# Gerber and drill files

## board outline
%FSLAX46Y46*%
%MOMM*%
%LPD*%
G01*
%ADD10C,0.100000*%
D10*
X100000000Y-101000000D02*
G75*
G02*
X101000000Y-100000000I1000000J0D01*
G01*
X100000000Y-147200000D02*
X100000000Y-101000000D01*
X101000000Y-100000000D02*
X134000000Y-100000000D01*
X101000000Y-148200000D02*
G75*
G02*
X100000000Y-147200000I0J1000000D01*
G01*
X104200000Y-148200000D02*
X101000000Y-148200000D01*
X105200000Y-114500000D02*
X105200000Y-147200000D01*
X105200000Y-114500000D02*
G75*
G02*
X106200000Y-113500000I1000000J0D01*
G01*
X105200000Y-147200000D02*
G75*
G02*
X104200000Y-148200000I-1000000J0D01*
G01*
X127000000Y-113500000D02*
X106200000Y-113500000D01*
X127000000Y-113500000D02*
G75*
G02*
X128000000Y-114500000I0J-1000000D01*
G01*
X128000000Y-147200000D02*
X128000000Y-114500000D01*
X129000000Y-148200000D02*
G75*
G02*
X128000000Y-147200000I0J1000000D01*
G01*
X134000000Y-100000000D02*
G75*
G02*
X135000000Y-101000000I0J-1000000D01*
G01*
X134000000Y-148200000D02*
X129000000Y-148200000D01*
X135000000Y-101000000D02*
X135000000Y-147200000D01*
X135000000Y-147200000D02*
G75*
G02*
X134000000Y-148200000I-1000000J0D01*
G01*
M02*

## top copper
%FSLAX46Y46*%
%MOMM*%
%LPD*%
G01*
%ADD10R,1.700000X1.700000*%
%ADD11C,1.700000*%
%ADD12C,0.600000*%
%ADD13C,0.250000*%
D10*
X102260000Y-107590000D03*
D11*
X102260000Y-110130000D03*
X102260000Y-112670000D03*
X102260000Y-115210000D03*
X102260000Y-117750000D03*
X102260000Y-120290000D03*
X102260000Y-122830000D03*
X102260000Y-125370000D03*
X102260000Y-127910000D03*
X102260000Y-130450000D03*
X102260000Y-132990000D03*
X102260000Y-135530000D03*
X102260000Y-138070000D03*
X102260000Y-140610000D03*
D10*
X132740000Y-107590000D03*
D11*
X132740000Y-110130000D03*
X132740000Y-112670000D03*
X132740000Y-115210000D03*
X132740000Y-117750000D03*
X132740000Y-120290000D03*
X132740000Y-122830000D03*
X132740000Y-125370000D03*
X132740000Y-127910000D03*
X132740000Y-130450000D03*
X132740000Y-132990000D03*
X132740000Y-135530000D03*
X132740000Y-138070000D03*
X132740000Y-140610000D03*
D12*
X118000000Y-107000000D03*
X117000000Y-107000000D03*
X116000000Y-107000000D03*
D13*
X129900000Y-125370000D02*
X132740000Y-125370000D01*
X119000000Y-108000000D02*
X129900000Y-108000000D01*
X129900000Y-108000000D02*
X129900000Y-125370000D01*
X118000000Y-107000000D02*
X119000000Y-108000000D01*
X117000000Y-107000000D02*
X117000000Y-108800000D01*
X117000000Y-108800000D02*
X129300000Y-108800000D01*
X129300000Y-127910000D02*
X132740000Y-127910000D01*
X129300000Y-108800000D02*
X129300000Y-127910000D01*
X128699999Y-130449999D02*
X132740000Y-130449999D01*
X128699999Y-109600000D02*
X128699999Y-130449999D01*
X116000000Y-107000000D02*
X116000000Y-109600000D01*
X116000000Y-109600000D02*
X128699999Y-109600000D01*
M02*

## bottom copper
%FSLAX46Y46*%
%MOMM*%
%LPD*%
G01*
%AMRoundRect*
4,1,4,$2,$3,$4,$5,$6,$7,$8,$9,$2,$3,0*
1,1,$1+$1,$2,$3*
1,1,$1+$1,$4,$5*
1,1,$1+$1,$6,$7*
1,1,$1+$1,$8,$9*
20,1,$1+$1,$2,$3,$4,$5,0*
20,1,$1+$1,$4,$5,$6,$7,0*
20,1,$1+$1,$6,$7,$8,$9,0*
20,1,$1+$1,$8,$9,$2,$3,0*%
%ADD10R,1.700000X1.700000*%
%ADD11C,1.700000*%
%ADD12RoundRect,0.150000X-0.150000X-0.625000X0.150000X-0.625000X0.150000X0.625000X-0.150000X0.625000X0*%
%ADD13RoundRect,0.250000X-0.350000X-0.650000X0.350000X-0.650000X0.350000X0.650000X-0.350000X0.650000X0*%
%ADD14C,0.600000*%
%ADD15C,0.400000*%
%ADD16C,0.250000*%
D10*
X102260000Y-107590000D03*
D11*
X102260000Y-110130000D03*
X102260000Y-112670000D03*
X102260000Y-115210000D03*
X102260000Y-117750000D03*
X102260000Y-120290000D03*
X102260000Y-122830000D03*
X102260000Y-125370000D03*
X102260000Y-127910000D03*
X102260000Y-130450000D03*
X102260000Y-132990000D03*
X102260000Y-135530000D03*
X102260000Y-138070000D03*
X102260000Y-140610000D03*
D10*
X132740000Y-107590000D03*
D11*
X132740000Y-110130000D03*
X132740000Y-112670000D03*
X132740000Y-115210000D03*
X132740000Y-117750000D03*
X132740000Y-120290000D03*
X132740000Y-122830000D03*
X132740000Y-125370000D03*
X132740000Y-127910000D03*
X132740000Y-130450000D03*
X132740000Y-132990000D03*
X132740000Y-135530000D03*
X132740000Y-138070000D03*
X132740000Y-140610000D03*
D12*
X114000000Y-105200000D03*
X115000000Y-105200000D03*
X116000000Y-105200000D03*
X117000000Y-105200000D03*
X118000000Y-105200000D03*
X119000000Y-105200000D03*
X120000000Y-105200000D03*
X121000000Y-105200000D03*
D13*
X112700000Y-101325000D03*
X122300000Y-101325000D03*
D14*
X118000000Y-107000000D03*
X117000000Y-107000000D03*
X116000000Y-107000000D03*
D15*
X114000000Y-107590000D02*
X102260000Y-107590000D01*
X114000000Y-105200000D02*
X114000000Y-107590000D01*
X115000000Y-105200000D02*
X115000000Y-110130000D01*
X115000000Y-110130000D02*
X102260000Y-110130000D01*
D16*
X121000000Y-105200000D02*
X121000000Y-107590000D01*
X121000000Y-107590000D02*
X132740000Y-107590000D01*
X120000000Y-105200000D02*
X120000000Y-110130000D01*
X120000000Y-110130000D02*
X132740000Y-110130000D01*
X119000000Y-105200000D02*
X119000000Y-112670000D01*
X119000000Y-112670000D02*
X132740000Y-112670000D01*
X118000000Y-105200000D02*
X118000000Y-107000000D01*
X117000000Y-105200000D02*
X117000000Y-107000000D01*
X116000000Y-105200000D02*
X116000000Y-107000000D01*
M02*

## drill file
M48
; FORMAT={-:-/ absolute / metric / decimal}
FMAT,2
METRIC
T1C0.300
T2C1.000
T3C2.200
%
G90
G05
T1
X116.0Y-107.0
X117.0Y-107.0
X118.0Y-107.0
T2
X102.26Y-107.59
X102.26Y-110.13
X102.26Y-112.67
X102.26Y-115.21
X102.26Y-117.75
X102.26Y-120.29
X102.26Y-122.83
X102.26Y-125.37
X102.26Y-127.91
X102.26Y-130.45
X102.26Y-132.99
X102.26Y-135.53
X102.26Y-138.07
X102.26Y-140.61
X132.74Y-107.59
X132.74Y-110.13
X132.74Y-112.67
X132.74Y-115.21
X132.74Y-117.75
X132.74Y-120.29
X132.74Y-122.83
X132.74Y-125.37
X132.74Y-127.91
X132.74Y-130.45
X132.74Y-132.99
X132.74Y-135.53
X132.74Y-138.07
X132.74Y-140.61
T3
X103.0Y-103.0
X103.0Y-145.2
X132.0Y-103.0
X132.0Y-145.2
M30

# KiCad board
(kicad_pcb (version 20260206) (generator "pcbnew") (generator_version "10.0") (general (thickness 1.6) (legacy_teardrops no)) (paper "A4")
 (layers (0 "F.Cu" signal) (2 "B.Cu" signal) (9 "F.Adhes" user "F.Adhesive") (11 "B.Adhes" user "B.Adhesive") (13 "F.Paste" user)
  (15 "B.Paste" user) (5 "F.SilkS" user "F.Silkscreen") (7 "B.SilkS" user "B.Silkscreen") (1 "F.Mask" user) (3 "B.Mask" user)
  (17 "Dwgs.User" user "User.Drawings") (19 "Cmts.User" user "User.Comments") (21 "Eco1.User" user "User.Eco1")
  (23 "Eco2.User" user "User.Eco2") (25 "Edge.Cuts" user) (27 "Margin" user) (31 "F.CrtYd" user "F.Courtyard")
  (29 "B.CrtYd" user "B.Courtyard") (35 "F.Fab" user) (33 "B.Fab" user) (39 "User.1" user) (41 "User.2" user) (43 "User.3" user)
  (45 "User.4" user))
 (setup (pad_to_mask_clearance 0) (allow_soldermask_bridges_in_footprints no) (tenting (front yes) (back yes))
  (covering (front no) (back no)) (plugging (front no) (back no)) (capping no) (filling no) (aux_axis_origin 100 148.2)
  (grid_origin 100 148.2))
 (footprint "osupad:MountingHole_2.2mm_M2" (layer "F.Cu") (at 132 145.2)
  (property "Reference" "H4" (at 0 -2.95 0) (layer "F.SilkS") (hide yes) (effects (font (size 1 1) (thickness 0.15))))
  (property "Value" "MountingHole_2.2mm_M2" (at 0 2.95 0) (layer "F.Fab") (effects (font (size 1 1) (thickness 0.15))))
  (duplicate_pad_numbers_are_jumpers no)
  (pad "" np_thru_hole circle (at 0 0) (size 2.2 2.2) (drill 2.2) (layers "*.Cu" "*.Mask")))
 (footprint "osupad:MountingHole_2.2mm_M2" (layer "F.Cu") (at 132 103)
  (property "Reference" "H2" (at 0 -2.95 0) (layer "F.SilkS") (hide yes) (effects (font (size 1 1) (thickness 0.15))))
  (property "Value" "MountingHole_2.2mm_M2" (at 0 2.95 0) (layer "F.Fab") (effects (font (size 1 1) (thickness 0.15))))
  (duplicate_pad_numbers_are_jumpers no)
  (pad "" np_thru_hole circle (at 0 0) (size 2.2 2.2) (drill 2.2) (layers "*.Cu" "*.Mask")))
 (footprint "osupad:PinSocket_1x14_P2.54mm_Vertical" (layer "F.Cu") (at 102.26 107.59)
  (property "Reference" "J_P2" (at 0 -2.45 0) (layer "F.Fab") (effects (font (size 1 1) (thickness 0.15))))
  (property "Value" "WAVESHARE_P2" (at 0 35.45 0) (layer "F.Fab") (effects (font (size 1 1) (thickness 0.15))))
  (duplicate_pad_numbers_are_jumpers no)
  (pad "1" thru_hole rect (at 0 0) (size 1.7 1.7) (drill 1) (layers "*.Cu" "*.Mask") (remove_unused_layers no) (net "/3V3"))
  (pad "2" thru_hole circle (at 0 2.54) (size 1.7 1.7) (drill 1) (layers "*.Cu" "*.Mask") (remove_unused_layers no) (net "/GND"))
  (pad "3" thru_hole circle (at 0 5.08) (size 1.7 1.7) (drill 1) (layers "*.Cu" "*.Mask") (remove_unused_layers no)
   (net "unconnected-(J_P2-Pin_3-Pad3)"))
  (pad "4" thru_hole circle (at 0 7.62) (size 1.7 1.7) (drill 1) (layers "*.Cu" "*.Mask") (remove_unused_layers no)
   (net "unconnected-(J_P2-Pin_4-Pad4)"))
  (pad "5" thru_hole circle (at 0 10.16) (size 1.7 1.7) (drill 1) (layers "*.Cu" "*.Mask") (remove_unused_layers no)
   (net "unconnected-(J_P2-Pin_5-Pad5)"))
  (pad "6" thru_hole circle (at 0 12.7) (size 1.7 1.7) (drill 1) (layers "*.Cu" "*.Mask") (remove_unused_layers no)
   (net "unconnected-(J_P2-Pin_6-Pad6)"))
  (pad "7" thru_hole circle (at 0 15.24) (size 1.7 1.7) (drill 1) (layers "*.Cu" "*.Mask") (remove_unused_layers no)
   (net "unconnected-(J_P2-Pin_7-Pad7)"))
  (pad "8" thru_hole circle (at 0 17.78) (size 1.7 1.7) (drill 1) (layers "*.Cu" "*.Mask") (remove_unused_layers no)
   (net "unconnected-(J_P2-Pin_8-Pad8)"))
  (pad "9" thru_hole circle (at 0 20.32) (size 1.7 1.7) (drill 1) (layers "*.Cu" "*.Mask") (remove_unused_layers no)
   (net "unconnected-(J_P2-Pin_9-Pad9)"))
  (pad "10" thru_hole circle (at 0 22.86) (size 1.7 1.7) (drill 1) (layers "*.Cu" "*.Mask") (remove_unused_layers no)
   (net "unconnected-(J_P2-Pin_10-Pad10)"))
  (pad "11" thru_hole circle (at 0 25.4) (size 1.7 1.7) (drill 1) (layers "*.Cu" "*.Mask") (remove_unused_layers no)
   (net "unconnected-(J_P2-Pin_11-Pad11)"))
  (pad "12" thru_hole circle (at 0 27.94) (size 1.7 1.7) (drill 1) (layers "*.Cu" "*.Mask") (remove_unused_layers no)
   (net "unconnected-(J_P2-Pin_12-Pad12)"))
  (pad "13" thru_hole circle (at 0 30.48) (size 1.7 1.7) (drill 1) (layers "*.Cu" "*.Mask") (remove_unused_layers no)
   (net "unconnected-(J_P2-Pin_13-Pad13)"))
  (pad "14" thru_hole circle (at 0 33.02) (size 1.7 1.7) (drill 1) (layers "*.Cu" "*.Mask") (remove_unused_layers no)
   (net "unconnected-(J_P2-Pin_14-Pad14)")))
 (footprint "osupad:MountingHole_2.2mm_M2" (layer "F.Cu") (at 103 103)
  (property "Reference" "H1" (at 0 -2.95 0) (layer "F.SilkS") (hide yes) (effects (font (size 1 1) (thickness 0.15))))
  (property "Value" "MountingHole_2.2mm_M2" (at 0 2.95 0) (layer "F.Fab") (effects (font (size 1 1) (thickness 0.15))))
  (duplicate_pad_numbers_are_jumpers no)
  (pad "" np_thru_hole circle (at 0 0) (size 2.2 2.2) (drill 2.2) (layers "*.Cu" "*.Mask")))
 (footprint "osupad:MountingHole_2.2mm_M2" (layer "F.Cu") (at 103 145.2)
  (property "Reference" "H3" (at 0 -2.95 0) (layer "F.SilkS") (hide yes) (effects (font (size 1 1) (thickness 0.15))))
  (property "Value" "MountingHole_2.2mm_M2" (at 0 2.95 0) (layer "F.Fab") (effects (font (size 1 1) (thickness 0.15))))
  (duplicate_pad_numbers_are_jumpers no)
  (pad "" np_thru_hole circle (at 0 0) (size 2.2 2.2) (drill 2.2) (layers "*.Cu" "*.Mask")))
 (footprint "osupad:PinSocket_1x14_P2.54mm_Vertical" (layer "F.Cu") (at 132.74 107.59)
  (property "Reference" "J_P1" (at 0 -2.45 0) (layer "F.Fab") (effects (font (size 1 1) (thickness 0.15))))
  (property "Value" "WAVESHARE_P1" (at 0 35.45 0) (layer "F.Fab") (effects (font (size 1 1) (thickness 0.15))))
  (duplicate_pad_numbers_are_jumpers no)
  (pad "1" thru_hole rect (at 0 0) (size 1.7 1.7) (drill 1) (layers "*.Cu" "*.Mask") (remove_unused_layers no) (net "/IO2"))
  (pad "2" thru_hole circle (at 0 2.54) (size 1.7 1.7) (drill 1) (layers "*.Cu" "*.Mask") (remove_unused_layers no) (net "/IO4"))
  (pad "3" thru_hole circle (at 0 5.08) (size 1.7 1.7) (drill 1) (layers "*.Cu" "*.Mask") (remove_unused_layers no) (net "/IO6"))
  (pad "4" thru_hole circle (at 0 7.62) (size 1.7 1.7) (drill 1) (layers "*.Cu" "*.Mask") (remove_unused_layers no)
   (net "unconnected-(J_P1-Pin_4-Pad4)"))
  (pad "5" thru_hole circle (at 0 10.16) (size 1.7 1.7) (drill 1) (layers "*.Cu" "*.Mask") (remove_unused_layers no)
   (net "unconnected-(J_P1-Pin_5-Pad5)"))
  (pad "6" thru_hole circle (at 0 12.7) (size 1.7 1.7) (drill 1) (layers "*.Cu" "*.Mask") (remove_unused_layers no)
   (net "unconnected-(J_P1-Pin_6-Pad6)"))
  (pad "7" thru_hole circle (at 0 15.24) (size 1.7 1.7) (drill 1) (layers "*.Cu" "*.Mask") (remove_unused_layers no)
   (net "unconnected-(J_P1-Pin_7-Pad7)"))
  (pad "8" thru_hole circle (at 0 17.78) (size 1.7 1.7) (drill 1) (layers "*.Cu" "*.Mask") (remove_unused_layers no) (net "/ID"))
  (pad "9" thru_hole circle (at 0 20.32) (size 1.7 1.7) (drill 1) (layers "*.Cu" "*.Mask") (remove_unused_layers no) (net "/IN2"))
  (pad "10" thru_hole circle (at 0 22.86) (size 1.7 1.7) (drill 1) (layers "*.Cu" "*.Mask") (remove_unused_layers no) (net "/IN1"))
  (pad "11" thru_hole circle (at 0 25.4) (size 1.7 1.7) (drill 1) (layers "*.Cu" "*.Mask") (remove_unused_layers no)
   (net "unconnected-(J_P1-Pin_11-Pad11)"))
  (pad "12" thru_hole circle (at 0 27.94) (size 1.7 1.7) (drill 1) (layers "*.Cu" "*.Mask") (remove_unused_layers no)
   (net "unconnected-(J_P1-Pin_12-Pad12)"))
  (pad "13" thru_hole circle (at 0 30.48) (size 1.7 1.7) (drill 1) (layers "*.Cu" "*.Mask") (remove_unused_layers no)
   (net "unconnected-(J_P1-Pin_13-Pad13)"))
  (pad "14" thru_hole circle (at 0 33.02) (size 1.7 1.7) (drill 1) (layers "*.Cu" "*.Mask") (remove_unused_layers no)
   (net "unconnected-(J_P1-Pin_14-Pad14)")))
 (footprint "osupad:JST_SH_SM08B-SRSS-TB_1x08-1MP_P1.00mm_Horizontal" (layer "B.Cu") (at 117.5 103.2)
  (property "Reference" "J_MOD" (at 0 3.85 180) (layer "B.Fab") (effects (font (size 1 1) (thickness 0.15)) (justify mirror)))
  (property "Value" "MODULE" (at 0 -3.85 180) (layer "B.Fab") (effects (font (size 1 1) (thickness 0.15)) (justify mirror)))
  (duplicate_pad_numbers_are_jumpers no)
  (pad "1" smd roundrect (at -3.5 2) (size 0.6 1.55) (layers "B.Cu" "B.Mask" "B.Paste") (roundrect_rratio 0.25) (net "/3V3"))
  (pad "2" smd roundrect (at -2.5 2) (size 0.6 1.55) (layers "B.Cu" "B.Mask" "B.Paste") (roundrect_rratio 0.25) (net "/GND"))
  (pad "3" smd roundrect (at -1.5 2) (size 0.6 1.55) (layers "B.Cu" "B.Mask" "B.Paste") (roundrect_rratio 0.25) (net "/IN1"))
  (pad "4" smd roundrect (at -0.5 2) (size 0.6 1.55) (layers "B.Cu" "B.Mask" "B.Paste") (roundrect_rratio 0.25) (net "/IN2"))
  (pad "5" smd roundrect (at 0.5 2) (size 0.6 1.55) (layers "B.Cu" "B.Mask" "B.Paste") (roundrect_rratio 0.25) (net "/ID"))
  (pad "6" smd roundrect (at 1.5 2) (size 0.6 1.55) (layers "B.Cu" "B.Mask" "B.Paste") (roundrect_rratio 0.25) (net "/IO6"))
  (pad "7" smd roundrect (at 2.5 2) (size 0.6 1.55) (layers "B.Cu" "B.Mask" "B.Paste") (roundrect_rratio 0.25) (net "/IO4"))
  (pad "8" smd roundrect (at 3.5 2) (size 0.6 1.55) (layers "B.Cu" "B.Mask" "B.Paste") (roundrect_rratio 0.25) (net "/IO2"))
  (pad "MP" smd roundrect (at -4.8 -1.875) (size 1.2 1.8) (layers "B.Cu" "B.Mask" "B.Paste") (roundrect_rratio 0.208333))
  (pad "MP" smd roundrect (at 4.8 -1.875) (size 1.2 1.8) (layers "B.Cu" "B.Mask" "B.Paste") (roundrect_rratio 0.208333)))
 (gr_arc (start 100 101) (mid 100.292893 100.292893) (end 101 100) (stroke (width 0.1) (type default)) (layer "Edge.Cuts"))
 (gr_line (start 100 147.2) (end 100 101) (stroke (width 0.1) (type default)) (layer "Edge.Cuts"))
 (gr_line (start 101 100) (end 134 100) (stroke (width 0.1) (type default)) (layer "Edge.Cuts"))
 (gr_arc (start 101 148.2) (mid 100.292893 147.907106) (end 100 147.2) (stroke (width 0.1) (type default)) (layer "Edge.Cuts"))
 (gr_line (start 104.2 148.2) (end 101 148.2) (stroke (width 0.1) (type default)) (layer "Edge.Cuts"))
 (gr_line (start 105.2 114.5) (end 105.2 147.2) (stroke (width 0.1) (type default)) (layer "Edge.Cuts"))
 (gr_arc (start 105.2 114.5) (mid 105.492893 113.792893) (end 106.2 113.5) (stroke (width 0.1) (type default)) (layer "Edge.Cuts"))
 (gr_arc (start 105.2 147.2) (mid 104.907106 147.907106) (end 104.2 148.2) (stroke (width 0.1) (type default)) (layer "Edge.Cuts"))
 (gr_line (start 127 113.5) (end 106.2 113.5) (stroke (width 0.1) (type default)) (layer "Edge.Cuts"))
 (gr_arc (start 127 113.5) (mid 127.707107 113.792893) (end 128 114.5) (stroke (width 0.1) (type default)) (layer "Edge.Cuts"))
 (gr_line (start 128 147.2) (end 128 114.5) (stroke (width 0.1) (type default)) (layer "Edge.Cuts"))
 (gr_arc (start 129 148.2) (mid 128.292893 147.907106) (end 128 147.2) (stroke (width 0.1) (type default)) (layer "Edge.Cuts"))
 (gr_arc (start 134 100) (mid 134.707106 100.292893) (end 135 101) (stroke (width 0.1) (type default)) (layer "Edge.Cuts"))
 (gr_line (start 134 148.2) (end 129 148.2) (stroke (width 0.1) (type default)) (layer "Edge.Cuts"))
 (gr_line (start 135 101) (end 135 147.2) (stroke (width 0.1) (type default)) (layer "Edge.Cuts"))
 (gr_arc (start 135 147.2) (mid 134.707106 147.907106) (end 134 148.2) (stroke (width 0.1) (type default)) (layer "Edge.Cuts"))
 (segment (start 114 107.59) (end 102.26 107.59) (width 0.4) (layer "B.Cu") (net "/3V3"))
 (segment (start 114 105.2) (end 114 107.59) (width 0.4) (layer "B.Cu") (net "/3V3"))
 (segment (start 115 105.2) (end 115 110.13) (width 0.4) (layer "B.Cu") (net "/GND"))
 (segment (start 115 110.13) (end 102.26 110.13) (width 0.4) (layer "B.Cu") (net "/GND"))
 (segment (start 121 105.2) (end 121 107.59) (width 0.25) (layer "B.Cu") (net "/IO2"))
 (segment (start 121 107.59) (end 132.74 107.59) (width 0.25) (layer "B.Cu") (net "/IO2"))
 (segment (start 120 105.2) (end 120 110.13) (width 0.25) (layer "B.Cu") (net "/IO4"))
 (segment (start 120 110.13) (end 132.74 110.13) (width 0.25) (layer "B.Cu") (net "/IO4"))
 (segment (start 119 105.2) (end 119 112.67) (width 0.25) (layer "B.Cu") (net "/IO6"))
 (segment (start 119 112.67) (end 132.74 112.67) (width 0.25) (layer "B.Cu") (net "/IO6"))
 (segment (start 129.9 125.37) (end 132.74 125.37) (width 0.25) (layer "F.Cu") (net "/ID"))
 (segment (start 119 108) (end 129.9 108) (width 0.25) (layer "F.Cu") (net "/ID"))
 (segment (start 129.9 108) (end 129.9 125.37) (width 0.25) (layer "F.Cu") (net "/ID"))
 (segment (start 118 107) (end 119 108) (width 0.25) (layer "F.Cu") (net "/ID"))
 (via (at 118 107) (size 0.6) (drill 0.3) (layers "F.Cu" "B.Cu") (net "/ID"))
 (segment (start 118 105.2) (end 118 107) (width 0.25) (layer "B.Cu") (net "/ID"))
 (segment (start 117 107) (end 117 108.8) (width 0.25) (layer "F.Cu") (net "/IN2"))
 (segment (start 117 108.8) (end 129.3 108.8) (width 0.25) (layer "F.Cu") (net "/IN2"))
 (segment (start 129.3 127.91) (end 132.74 127.91) (width 0.25) (layer "F.Cu") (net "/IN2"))
 (segment (start 129.3 108.8) (end 129.3 127.91) (width 0.25) (layer "F.Cu") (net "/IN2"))
 (via (at 117 107) (size 0.6) (drill 0.3) (layers "F.Cu" "B.Cu") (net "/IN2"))
 (segment (start 117 105.2) (end 117 107) (width 0.25) (layer "B.Cu") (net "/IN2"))
 (segment (start 128.699999 130.449999) (end 132.74 130.449999) (width 0.25) (layer "F.Cu") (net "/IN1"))
 (segment (start 128.699999 109.6) (end 128.699999 130.449999) (width 0.25) (layer "F.Cu") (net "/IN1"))
 (segment (start 116 107) (end 116 109.6) (width 0.25) (layer "F.Cu") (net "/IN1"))
 (segment (start 116 109.6) (end 128.699999 109.6) (width 0.25) (layer "F.Cu") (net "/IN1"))
 (via (at 116 107) (size 0.6) (drill 0.3) (layers "F.Cu" "B.Cu") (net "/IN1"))
 (segment (start 116 105.2) (end 116 107) (width 0.25) (layer "B.Cu") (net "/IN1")))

